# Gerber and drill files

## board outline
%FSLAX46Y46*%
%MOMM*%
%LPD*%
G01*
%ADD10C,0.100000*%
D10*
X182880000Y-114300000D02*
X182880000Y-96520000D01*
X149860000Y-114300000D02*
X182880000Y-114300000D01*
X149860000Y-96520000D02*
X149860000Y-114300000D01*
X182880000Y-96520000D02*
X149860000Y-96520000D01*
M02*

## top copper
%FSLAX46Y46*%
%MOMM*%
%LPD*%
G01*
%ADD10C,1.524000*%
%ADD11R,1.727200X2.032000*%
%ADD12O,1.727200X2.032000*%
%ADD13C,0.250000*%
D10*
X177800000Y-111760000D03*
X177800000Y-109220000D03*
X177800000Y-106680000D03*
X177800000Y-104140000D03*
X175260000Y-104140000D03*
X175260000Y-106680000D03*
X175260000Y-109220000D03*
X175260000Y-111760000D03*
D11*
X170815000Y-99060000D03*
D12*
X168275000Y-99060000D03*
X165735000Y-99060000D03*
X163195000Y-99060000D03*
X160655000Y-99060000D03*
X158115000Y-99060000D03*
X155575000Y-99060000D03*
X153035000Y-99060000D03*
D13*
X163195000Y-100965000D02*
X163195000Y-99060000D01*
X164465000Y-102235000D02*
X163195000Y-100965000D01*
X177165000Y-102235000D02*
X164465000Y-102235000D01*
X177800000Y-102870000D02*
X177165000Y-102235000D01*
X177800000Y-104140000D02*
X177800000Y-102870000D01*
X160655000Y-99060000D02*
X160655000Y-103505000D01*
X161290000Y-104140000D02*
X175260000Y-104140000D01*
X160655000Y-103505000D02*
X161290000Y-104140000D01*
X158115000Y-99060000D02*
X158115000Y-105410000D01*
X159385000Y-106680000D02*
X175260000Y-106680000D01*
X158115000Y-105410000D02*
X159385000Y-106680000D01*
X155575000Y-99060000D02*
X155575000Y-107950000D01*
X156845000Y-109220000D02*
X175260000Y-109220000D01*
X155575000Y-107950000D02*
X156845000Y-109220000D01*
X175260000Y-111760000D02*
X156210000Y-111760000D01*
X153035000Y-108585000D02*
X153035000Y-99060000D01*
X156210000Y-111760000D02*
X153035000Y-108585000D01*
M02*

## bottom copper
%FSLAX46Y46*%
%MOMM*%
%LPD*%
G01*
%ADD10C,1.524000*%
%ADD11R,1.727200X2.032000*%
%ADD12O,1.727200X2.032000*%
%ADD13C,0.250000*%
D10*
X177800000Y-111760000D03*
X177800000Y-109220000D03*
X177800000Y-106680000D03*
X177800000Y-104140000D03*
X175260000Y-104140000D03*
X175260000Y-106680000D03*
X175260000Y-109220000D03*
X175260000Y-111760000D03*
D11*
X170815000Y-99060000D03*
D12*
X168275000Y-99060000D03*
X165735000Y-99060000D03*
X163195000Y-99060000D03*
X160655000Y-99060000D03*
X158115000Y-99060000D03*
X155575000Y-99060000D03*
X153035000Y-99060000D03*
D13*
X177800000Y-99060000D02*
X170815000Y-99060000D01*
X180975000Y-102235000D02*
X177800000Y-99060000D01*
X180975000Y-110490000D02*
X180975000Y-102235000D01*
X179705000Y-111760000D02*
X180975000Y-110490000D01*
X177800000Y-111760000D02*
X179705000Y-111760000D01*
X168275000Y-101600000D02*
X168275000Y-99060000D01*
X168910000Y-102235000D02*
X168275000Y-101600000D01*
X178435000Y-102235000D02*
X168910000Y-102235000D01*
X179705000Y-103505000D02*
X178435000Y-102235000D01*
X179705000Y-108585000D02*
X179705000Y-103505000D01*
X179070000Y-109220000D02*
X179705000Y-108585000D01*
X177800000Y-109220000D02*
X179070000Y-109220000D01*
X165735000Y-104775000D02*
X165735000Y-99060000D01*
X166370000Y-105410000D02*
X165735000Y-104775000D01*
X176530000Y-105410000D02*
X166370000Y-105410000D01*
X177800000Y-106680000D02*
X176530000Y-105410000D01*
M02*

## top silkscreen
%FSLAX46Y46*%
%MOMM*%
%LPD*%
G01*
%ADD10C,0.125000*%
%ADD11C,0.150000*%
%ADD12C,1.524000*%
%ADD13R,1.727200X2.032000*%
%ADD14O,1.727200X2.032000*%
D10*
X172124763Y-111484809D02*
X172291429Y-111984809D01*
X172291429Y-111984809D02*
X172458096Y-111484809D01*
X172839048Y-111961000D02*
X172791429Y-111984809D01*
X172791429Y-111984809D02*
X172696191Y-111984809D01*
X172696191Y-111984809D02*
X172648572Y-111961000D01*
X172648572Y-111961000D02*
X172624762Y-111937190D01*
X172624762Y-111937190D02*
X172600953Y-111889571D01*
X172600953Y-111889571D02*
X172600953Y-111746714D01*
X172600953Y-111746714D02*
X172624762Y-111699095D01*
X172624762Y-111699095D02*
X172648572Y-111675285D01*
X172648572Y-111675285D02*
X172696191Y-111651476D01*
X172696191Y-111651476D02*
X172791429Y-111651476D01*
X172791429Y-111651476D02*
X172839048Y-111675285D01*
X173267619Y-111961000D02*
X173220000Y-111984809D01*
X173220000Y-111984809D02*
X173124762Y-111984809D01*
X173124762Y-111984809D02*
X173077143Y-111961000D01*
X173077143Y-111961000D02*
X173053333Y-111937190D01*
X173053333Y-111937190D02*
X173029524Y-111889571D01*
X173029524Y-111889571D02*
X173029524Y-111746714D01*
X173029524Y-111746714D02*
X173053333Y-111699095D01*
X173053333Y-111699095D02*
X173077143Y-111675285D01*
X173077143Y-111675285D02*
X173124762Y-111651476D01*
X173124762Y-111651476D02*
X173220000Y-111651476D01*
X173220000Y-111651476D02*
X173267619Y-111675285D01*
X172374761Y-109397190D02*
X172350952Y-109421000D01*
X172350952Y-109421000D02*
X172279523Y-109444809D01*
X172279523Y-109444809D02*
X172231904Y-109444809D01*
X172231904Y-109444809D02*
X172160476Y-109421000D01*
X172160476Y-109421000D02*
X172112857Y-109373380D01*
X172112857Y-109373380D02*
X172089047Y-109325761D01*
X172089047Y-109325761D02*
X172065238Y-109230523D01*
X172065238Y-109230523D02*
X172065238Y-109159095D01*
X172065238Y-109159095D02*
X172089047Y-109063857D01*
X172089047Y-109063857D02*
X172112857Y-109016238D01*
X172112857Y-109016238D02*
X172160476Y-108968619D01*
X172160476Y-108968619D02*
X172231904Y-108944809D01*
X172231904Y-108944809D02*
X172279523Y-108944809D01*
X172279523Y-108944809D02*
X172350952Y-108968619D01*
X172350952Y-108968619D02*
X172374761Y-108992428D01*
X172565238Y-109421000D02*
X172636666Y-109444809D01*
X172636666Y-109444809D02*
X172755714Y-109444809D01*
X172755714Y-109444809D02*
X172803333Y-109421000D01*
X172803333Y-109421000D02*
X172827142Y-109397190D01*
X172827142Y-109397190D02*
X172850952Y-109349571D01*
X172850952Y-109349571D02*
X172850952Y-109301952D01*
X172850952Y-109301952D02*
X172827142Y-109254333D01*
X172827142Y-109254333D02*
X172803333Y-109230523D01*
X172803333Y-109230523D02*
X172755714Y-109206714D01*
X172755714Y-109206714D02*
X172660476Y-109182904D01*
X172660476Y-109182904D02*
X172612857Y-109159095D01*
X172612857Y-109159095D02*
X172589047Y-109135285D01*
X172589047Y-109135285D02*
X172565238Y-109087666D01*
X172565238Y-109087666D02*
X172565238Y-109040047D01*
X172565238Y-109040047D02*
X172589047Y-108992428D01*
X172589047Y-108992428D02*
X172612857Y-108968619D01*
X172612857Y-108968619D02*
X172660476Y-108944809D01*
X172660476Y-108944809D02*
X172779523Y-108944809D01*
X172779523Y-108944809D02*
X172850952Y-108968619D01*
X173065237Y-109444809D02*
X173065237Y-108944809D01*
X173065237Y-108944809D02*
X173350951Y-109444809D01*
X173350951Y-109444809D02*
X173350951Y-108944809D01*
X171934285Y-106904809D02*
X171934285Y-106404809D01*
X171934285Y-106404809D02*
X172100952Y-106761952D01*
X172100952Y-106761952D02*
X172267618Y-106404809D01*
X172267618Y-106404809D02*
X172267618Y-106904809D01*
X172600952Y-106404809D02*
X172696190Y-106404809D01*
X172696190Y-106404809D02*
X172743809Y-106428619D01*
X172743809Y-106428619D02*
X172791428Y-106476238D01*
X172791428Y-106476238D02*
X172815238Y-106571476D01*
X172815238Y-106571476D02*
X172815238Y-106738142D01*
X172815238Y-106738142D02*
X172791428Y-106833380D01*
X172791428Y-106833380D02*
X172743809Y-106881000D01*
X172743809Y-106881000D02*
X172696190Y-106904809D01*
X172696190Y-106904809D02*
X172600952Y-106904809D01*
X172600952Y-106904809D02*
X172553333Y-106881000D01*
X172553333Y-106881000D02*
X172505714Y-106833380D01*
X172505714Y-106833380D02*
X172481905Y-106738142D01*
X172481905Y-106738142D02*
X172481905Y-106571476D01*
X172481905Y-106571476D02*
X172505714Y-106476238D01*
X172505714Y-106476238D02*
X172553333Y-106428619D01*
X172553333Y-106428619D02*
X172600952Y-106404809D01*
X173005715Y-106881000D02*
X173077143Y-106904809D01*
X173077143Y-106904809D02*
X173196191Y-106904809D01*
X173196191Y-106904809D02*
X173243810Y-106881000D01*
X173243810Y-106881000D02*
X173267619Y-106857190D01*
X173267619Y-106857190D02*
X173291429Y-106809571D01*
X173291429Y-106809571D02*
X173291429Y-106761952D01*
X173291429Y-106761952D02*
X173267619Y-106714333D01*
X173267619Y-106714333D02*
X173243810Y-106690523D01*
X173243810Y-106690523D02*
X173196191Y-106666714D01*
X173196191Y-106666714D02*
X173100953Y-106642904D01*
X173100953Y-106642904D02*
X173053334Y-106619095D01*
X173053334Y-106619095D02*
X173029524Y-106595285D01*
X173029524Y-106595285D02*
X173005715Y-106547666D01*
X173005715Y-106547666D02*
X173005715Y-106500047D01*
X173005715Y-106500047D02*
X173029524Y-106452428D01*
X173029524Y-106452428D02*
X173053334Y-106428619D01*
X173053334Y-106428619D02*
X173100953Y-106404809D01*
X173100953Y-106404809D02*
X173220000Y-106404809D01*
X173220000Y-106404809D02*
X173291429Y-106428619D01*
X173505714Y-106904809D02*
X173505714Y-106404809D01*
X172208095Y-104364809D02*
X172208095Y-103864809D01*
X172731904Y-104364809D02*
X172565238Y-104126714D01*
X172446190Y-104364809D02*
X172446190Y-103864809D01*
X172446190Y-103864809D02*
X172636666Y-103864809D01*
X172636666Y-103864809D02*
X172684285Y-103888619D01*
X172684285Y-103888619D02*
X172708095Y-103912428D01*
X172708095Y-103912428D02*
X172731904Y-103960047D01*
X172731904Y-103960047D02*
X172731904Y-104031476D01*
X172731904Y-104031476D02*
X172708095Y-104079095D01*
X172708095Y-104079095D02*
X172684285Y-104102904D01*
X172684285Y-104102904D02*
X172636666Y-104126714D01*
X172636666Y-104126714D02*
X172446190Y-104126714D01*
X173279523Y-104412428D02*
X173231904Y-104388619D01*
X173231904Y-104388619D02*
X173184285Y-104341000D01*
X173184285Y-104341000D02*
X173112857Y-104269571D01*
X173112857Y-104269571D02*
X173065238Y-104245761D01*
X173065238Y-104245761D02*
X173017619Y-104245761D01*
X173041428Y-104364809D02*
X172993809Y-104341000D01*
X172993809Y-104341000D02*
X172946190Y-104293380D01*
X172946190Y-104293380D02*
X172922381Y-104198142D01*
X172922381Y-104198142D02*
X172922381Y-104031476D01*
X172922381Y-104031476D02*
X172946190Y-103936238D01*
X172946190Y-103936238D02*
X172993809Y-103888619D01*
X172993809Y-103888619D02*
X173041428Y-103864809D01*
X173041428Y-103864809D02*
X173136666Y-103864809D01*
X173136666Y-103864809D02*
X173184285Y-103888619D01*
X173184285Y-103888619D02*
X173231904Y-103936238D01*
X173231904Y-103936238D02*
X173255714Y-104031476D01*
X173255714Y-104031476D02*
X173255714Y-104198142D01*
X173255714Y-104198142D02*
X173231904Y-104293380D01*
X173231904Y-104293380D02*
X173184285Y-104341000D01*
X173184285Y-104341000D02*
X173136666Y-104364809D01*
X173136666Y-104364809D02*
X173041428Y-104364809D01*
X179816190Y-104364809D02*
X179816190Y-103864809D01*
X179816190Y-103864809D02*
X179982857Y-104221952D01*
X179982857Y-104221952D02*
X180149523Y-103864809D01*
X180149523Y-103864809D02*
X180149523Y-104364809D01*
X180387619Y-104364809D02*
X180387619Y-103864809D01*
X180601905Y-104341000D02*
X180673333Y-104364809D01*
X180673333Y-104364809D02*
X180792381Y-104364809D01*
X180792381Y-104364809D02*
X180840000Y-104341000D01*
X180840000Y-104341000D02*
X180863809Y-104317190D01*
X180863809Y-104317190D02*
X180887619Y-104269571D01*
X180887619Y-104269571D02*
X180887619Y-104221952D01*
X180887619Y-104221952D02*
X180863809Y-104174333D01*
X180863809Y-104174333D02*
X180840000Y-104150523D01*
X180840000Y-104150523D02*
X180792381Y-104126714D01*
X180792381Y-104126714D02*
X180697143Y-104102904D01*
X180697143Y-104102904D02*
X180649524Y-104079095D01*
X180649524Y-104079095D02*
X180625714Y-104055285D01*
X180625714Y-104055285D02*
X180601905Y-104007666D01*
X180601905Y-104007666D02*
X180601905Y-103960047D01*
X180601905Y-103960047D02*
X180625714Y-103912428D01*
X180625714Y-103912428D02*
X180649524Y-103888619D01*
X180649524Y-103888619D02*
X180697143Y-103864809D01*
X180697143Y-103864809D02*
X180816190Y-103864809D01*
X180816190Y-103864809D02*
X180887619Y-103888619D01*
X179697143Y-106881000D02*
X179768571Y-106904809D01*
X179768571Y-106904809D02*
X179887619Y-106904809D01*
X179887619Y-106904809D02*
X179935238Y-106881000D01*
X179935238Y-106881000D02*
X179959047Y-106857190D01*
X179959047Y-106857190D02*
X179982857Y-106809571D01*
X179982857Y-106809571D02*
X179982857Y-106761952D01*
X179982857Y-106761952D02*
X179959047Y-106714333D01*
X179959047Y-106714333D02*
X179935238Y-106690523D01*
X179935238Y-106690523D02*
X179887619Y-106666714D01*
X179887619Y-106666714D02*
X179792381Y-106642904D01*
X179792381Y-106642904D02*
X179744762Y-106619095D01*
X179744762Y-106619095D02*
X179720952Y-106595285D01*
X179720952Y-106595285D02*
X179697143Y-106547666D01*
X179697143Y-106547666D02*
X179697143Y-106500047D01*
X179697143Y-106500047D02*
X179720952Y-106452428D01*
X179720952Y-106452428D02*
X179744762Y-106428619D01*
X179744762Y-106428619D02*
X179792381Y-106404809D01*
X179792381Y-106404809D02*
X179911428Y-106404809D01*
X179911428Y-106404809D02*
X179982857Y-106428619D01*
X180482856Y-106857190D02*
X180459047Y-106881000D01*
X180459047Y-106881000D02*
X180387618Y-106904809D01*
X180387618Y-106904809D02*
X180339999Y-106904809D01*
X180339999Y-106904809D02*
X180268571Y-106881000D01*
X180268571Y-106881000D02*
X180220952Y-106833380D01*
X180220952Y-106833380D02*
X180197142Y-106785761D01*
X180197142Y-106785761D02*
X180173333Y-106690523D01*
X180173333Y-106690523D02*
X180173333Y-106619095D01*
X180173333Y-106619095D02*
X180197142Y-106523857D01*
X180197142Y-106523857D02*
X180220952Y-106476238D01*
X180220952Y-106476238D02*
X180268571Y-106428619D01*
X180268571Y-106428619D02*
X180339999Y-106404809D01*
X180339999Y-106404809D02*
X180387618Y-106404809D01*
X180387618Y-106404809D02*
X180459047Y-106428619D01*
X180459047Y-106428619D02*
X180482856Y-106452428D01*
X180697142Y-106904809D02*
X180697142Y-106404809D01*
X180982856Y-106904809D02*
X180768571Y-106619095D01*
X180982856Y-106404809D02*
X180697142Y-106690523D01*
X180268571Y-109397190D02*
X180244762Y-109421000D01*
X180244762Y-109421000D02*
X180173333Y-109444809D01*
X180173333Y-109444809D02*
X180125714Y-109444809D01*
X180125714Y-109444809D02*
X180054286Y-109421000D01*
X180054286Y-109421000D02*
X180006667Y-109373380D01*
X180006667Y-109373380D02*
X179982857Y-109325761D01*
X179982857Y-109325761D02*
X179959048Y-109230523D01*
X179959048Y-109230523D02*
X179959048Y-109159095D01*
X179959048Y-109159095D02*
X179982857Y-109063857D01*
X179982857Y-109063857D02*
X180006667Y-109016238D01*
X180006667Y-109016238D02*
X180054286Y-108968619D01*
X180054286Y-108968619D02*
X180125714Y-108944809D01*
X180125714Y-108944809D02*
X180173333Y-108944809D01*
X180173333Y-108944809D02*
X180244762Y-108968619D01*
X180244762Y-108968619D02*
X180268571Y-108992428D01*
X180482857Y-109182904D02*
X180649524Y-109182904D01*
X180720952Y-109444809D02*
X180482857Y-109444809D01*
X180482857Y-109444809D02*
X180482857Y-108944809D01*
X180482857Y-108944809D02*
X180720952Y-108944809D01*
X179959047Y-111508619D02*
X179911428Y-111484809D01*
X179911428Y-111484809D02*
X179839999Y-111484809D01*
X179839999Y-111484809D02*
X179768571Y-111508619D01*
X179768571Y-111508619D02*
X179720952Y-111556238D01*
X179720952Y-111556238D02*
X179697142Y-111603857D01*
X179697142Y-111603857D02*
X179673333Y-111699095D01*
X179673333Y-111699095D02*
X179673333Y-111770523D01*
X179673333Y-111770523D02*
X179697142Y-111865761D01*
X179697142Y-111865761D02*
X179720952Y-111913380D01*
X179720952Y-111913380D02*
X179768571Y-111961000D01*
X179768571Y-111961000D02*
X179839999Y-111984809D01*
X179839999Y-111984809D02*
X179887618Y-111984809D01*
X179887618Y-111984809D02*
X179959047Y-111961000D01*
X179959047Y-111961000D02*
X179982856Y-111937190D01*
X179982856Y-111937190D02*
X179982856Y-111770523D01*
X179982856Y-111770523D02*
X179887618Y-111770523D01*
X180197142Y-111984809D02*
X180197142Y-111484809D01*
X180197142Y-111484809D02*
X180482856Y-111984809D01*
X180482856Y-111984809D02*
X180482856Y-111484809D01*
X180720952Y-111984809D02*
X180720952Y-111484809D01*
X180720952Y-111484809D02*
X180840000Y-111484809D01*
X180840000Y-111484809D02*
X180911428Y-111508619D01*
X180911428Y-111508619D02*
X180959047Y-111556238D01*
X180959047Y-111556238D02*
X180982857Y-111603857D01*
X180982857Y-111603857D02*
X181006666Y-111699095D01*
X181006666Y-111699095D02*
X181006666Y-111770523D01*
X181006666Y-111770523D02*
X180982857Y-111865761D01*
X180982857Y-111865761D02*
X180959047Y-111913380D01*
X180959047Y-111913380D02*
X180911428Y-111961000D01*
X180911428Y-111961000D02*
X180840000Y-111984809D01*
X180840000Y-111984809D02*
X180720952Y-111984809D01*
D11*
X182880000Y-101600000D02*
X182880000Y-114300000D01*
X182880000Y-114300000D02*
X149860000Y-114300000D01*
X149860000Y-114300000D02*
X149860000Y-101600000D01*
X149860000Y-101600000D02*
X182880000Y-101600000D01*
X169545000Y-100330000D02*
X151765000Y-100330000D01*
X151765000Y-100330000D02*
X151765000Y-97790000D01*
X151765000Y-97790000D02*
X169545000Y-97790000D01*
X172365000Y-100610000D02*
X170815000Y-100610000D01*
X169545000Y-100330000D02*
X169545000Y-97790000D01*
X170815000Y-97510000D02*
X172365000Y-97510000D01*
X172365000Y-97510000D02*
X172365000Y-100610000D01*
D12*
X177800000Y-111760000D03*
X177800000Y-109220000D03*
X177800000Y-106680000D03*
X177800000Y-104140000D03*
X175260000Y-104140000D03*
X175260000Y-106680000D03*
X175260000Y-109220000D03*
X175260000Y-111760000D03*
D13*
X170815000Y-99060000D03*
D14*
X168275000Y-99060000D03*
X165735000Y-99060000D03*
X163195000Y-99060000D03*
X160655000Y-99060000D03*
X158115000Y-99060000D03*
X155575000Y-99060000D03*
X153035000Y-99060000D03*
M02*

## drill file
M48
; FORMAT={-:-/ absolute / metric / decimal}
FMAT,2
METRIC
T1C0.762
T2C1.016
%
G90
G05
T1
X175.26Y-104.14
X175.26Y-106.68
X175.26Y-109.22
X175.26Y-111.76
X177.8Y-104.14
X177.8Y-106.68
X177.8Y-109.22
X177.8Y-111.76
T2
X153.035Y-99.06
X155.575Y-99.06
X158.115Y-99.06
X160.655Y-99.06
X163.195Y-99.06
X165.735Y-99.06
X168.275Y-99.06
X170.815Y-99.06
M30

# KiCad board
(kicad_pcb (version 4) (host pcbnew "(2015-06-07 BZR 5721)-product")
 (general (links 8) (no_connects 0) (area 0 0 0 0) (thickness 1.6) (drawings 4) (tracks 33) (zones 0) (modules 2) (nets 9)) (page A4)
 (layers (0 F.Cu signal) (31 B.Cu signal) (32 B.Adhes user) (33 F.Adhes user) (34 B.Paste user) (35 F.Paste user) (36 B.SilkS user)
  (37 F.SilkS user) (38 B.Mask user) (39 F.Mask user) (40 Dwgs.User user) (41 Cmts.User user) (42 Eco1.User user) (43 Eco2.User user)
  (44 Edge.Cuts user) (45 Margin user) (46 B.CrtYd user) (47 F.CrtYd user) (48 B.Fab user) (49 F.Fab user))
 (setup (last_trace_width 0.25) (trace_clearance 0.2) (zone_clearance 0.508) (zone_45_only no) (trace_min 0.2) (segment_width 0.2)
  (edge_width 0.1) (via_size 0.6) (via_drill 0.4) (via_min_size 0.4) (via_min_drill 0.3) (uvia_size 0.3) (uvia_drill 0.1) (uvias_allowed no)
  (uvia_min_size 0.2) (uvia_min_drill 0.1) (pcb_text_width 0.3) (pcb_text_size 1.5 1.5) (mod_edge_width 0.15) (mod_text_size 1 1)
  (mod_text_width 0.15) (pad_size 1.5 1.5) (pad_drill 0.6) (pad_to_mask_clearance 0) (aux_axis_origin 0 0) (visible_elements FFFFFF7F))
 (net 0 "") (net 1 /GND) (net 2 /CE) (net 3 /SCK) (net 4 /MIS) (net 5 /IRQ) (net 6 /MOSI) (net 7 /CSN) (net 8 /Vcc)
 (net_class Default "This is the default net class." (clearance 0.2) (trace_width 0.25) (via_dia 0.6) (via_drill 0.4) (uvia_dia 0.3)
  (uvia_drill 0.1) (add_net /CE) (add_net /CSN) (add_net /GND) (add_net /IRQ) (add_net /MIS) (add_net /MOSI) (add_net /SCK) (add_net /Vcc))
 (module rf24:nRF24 (layer F.Cu) (at 170.18 109.22)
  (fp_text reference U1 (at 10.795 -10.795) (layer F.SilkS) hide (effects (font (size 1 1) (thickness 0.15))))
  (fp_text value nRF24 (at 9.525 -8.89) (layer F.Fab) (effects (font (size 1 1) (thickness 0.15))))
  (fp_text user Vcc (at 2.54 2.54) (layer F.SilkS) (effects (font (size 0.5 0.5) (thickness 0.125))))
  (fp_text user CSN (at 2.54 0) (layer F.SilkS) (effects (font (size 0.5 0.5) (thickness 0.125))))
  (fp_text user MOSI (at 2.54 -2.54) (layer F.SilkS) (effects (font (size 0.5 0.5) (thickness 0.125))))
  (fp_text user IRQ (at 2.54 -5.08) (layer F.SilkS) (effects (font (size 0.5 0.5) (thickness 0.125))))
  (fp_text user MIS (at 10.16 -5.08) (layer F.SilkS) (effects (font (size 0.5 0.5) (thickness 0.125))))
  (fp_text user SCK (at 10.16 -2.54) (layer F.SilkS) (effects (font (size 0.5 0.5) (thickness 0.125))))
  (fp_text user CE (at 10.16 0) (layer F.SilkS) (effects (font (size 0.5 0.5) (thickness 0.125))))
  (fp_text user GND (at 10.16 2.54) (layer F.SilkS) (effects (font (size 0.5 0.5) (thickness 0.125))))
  (fp_line (start 12.7 -7.62) (end 12.7 5.08) (layer F.SilkS) (width 0.15))
  (fp_line (start 12.7 5.08) (end -20.32 5.08) (layer F.SilkS) (width 0.15))
  (fp_line (start -20.32 5.08) (end -20.32 -7.62) (layer F.SilkS) (width 0.15))
  (fp_line (start -20.32 -7.62) (end 12.7 -7.62) (layer F.SilkS) (width 0.15))
  (pad 0 thru_hole circle (at 7.62 2.54) (size 1.524 1.524) (drill 0.762) (layers *.Cu *.Mask F.SilkS) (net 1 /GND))
  (pad 1 thru_hole circle (at 7.62 0) (size 1.524 1.524) (drill 0.762) (layers *.Cu *.Mask F.SilkS) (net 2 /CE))
  (pad 2 thru_hole circle (at 7.62 -2.54) (size 1.524 1.524) (drill 0.762) (layers *.Cu *.Mask F.SilkS) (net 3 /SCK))
  (pad 3 thru_hole circle (at 7.62 -5.08) (size 1.524 1.524) (drill 0.762) (layers *.Cu *.Mask F.SilkS) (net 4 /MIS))
  (pad 4 thru_hole circle (at 5.08 -5.08) (size 1.524 1.524) (drill 0.762) (layers *.Cu *.Mask F.SilkS) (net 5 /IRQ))
  (pad 5 thru_hole circle (at 5.08 -2.54) (size 1.524 1.524) (drill 0.762) (layers *.Cu *.Mask F.SilkS) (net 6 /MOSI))
  (pad 6 thru_hole circle (at 5.08 0) (size 1.524 1.524) (drill 0.762) (layers *.Cu *.Mask F.SilkS) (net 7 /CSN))
  (pad 7 thru_hole circle (at 5.08 2.54) (size 1.524 1.524) (drill 0.762) (layers *.Cu *.Mask F.SilkS) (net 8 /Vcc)))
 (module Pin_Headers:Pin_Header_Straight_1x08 (layer F.Cu) (at 170.815 99.06 270)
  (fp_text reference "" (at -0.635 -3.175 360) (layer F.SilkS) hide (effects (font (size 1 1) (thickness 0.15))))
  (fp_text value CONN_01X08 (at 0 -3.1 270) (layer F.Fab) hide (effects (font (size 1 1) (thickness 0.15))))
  (fp_line (start 1.27 1.27) (end 1.27 19.05) (layer F.SilkS) (width 0.15))
  (fp_line (start 1.27 19.05) (end -1.27 19.05) (layer F.SilkS) (width 0.15))
  (fp_line (start -1.27 19.05) (end -1.27 1.27) (layer F.SilkS) (width 0.15))
  (fp_line (start 1.55 -1.55) (end 1.55 0) (layer F.SilkS) (width 0.15))
  (fp_line (start 1.27 1.27) (end -1.27 1.27) (layer F.SilkS) (width 0.15))
  (fp_line (start -1.55 0) (end -1.55 -1.55) (layer F.SilkS) (width 0.15))
  (fp_line (start -1.55 -1.55) (end 1.55 -1.55) (layer F.SilkS) (width 0.15))
  (pad 1 thru_hole rect (at 0 0 270) (size 2.032 1.7272) (drill 1.016) (layers *.Cu *.Mask F.SilkS) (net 1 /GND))
  (pad 2 thru_hole oval (at 0 2.54 270) (size 2.032 1.7272) (drill 1.016) (layers *.Cu *.Mask F.SilkS) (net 2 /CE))
  (pad 3 thru_hole oval (at 0 5.08 270) (size 2.032 1.7272) (drill 1.016) (layers *.Cu *.Mask F.SilkS) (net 3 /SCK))
  (pad 4 thru_hole oval (at 0 7.62 270) (size 2.032 1.7272) (drill 1.016) (layers *.Cu *.Mask F.SilkS) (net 4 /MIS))
  (pad 5 thru_hole oval (at 0 10.16 270) (size 2.032 1.7272) (drill 1.016) (layers *.Cu *.Mask F.SilkS) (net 5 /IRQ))
  (pad 6 thru_hole oval (at 0 12.7 270) (size 2.032 1.7272) (drill 1.016) (layers *.Cu *.Mask F.SilkS) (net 6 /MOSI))
  (pad 7 thru_hole oval (at 0 15.24 270) (size 2.032 1.7272) (drill 1.016) (layers *.Cu *.Mask F.SilkS) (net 7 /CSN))
  (pad 8 thru_hole oval (at 0 17.78 270) (size 2.032 1.7272) (drill 1.016) (layers *.Cu *.Mask F.SilkS) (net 8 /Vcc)))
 (gr_line (start 182.88 114.3) (end 182.88 96.52) (angle 90) (layer Edge.Cuts) (width 0.1))
 (gr_line (start 149.86 114.3) (end 182.88 114.3) (angle 90) (layer Edge.Cuts) (width 0.1))
 (gr_line (start 149.86 96.52) (end 149.86 114.3) (angle 90) (layer Edge.Cuts) (width 0.1))
 (gr_line (start 182.88 96.52) (end 149.86 96.52) (angle 90) (layer Edge.Cuts) (width 0.1))
 (segment (start 177.8 99.06) (end 170.815 99.06) (width 0.25) (layer B.Cu) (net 1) (status 20))
 (segment (start 180.975 102.235) (end 177.8 99.06) (width 0.25) (layer B.Cu) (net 1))
 (segment (start 180.975 110.49) (end 180.975 102.235) (width 0.25) (layer B.Cu) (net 1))
 (segment (start 179.705 111.76) (end 180.975 110.49) (width 0.25) (layer B.Cu) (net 1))
 (segment (start 177.8 111.76) (end 179.705 111.76) (width 0.25) (layer B.Cu) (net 1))
 (segment (start 168.275 101.6) (end 168.275 99.06) (width 0.25) (layer B.Cu) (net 2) (status 20))
 (segment (start 168.91 102.235) (end 168.275 101.6) (width 0.25) (layer B.Cu) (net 2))
 (segment (start 178.435 102.235) (end 168.91 102.235) (width 0.25) (layer B.Cu) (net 2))
 (segment (start 179.705 103.505) (end 178.435 102.235) (width 0.25) (layer B.Cu) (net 2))
 (segment (start 179.705 108.585) (end 179.705 103.505) (width 0.25) (layer B.Cu) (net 2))
 (segment (start 179.07 109.22) (end 179.705 108.585) (width 0.25) (layer B.Cu) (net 2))
 (segment (start 177.8 109.22) (end 179.07 109.22) (width 0.25) (layer B.Cu) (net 2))
 (segment (start 165.735 104.775) (end 165.735 99.06) (width 0.25) (layer B.Cu) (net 3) (status 20))
 (segment (start 166.37 105.41) (end 165.735 104.775) (width 0.25) (layer B.Cu) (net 3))
 (segment (start 176.53 105.41) (end 166.37 105.41) (width 0.25) (layer B.Cu) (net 3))
 (segment (start 177.8 106.68) (end 176.53 105.41) (width 0.25) (layer B.Cu) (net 3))
 (segment (start 163.195 100.965) (end 163.195 99.06) (width 0.25) (layer F.Cu) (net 4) (status 20))
 (segment (start 164.465 102.235) (end 163.195 100.965) (width 0.25) (layer F.Cu) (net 4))
 (segment (start 177.165 102.235) (end 164.465 102.235) (width 0.25) (layer F.Cu) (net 4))
 (segment (start 177.8 102.87) (end 177.165 102.235) (width 0.25) (layer F.Cu) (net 4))
 (segment (start 177.8 104.14) (end 177.8 102.87) (width 0.25) (layer F.Cu) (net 4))
 (segment (start 160.655 99.06) (end 160.655 103.505) (width 0.25) (layer F.Cu) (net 5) (status 10))
 (segment (start 161.29 104.14) (end 175.26 104.14) (width 0.25) (layer F.Cu) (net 5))
 (segment (start 160.655 103.505) (end 161.29 104.14) (width 0.25) (layer F.Cu) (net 5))
 (segment (start 158.115 99.06) (end 158.115 105.41) (width 0.25) (layer F.Cu) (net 6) (status 10))
 (segment (start 159.385 106.68) (end 175.26 106.68) (width 0.25) (layer F.Cu) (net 6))
 (segment (start 158.115 105.41) (end 159.385 106.68) (width 0.25) (layer F.Cu) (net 6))
 (segment (start 155.575 99.06) (end 155.575 107.95) (width 0.25) (layer F.Cu) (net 7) (status 10))
 (segment (start 156.845 109.22) (end 175.26 109.22) (width 0.25) (layer F.Cu) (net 7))
 (segment (start 155.575 107.95) (end 156.845 109.22) (width 0.25) (layer F.Cu) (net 7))
 (segment (start 175.26 111.76) (end 156.21 111.76) (width 0.25) (layer F.Cu) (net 8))
 (segment (start 153.035 108.585) (end 153.035 99.06) (width 0.25) (layer F.Cu) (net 8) (status 20))
 (segment (start 156.21 111.76) (end 153.035 108.585) (width 0.25) (layer F.Cu) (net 8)))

